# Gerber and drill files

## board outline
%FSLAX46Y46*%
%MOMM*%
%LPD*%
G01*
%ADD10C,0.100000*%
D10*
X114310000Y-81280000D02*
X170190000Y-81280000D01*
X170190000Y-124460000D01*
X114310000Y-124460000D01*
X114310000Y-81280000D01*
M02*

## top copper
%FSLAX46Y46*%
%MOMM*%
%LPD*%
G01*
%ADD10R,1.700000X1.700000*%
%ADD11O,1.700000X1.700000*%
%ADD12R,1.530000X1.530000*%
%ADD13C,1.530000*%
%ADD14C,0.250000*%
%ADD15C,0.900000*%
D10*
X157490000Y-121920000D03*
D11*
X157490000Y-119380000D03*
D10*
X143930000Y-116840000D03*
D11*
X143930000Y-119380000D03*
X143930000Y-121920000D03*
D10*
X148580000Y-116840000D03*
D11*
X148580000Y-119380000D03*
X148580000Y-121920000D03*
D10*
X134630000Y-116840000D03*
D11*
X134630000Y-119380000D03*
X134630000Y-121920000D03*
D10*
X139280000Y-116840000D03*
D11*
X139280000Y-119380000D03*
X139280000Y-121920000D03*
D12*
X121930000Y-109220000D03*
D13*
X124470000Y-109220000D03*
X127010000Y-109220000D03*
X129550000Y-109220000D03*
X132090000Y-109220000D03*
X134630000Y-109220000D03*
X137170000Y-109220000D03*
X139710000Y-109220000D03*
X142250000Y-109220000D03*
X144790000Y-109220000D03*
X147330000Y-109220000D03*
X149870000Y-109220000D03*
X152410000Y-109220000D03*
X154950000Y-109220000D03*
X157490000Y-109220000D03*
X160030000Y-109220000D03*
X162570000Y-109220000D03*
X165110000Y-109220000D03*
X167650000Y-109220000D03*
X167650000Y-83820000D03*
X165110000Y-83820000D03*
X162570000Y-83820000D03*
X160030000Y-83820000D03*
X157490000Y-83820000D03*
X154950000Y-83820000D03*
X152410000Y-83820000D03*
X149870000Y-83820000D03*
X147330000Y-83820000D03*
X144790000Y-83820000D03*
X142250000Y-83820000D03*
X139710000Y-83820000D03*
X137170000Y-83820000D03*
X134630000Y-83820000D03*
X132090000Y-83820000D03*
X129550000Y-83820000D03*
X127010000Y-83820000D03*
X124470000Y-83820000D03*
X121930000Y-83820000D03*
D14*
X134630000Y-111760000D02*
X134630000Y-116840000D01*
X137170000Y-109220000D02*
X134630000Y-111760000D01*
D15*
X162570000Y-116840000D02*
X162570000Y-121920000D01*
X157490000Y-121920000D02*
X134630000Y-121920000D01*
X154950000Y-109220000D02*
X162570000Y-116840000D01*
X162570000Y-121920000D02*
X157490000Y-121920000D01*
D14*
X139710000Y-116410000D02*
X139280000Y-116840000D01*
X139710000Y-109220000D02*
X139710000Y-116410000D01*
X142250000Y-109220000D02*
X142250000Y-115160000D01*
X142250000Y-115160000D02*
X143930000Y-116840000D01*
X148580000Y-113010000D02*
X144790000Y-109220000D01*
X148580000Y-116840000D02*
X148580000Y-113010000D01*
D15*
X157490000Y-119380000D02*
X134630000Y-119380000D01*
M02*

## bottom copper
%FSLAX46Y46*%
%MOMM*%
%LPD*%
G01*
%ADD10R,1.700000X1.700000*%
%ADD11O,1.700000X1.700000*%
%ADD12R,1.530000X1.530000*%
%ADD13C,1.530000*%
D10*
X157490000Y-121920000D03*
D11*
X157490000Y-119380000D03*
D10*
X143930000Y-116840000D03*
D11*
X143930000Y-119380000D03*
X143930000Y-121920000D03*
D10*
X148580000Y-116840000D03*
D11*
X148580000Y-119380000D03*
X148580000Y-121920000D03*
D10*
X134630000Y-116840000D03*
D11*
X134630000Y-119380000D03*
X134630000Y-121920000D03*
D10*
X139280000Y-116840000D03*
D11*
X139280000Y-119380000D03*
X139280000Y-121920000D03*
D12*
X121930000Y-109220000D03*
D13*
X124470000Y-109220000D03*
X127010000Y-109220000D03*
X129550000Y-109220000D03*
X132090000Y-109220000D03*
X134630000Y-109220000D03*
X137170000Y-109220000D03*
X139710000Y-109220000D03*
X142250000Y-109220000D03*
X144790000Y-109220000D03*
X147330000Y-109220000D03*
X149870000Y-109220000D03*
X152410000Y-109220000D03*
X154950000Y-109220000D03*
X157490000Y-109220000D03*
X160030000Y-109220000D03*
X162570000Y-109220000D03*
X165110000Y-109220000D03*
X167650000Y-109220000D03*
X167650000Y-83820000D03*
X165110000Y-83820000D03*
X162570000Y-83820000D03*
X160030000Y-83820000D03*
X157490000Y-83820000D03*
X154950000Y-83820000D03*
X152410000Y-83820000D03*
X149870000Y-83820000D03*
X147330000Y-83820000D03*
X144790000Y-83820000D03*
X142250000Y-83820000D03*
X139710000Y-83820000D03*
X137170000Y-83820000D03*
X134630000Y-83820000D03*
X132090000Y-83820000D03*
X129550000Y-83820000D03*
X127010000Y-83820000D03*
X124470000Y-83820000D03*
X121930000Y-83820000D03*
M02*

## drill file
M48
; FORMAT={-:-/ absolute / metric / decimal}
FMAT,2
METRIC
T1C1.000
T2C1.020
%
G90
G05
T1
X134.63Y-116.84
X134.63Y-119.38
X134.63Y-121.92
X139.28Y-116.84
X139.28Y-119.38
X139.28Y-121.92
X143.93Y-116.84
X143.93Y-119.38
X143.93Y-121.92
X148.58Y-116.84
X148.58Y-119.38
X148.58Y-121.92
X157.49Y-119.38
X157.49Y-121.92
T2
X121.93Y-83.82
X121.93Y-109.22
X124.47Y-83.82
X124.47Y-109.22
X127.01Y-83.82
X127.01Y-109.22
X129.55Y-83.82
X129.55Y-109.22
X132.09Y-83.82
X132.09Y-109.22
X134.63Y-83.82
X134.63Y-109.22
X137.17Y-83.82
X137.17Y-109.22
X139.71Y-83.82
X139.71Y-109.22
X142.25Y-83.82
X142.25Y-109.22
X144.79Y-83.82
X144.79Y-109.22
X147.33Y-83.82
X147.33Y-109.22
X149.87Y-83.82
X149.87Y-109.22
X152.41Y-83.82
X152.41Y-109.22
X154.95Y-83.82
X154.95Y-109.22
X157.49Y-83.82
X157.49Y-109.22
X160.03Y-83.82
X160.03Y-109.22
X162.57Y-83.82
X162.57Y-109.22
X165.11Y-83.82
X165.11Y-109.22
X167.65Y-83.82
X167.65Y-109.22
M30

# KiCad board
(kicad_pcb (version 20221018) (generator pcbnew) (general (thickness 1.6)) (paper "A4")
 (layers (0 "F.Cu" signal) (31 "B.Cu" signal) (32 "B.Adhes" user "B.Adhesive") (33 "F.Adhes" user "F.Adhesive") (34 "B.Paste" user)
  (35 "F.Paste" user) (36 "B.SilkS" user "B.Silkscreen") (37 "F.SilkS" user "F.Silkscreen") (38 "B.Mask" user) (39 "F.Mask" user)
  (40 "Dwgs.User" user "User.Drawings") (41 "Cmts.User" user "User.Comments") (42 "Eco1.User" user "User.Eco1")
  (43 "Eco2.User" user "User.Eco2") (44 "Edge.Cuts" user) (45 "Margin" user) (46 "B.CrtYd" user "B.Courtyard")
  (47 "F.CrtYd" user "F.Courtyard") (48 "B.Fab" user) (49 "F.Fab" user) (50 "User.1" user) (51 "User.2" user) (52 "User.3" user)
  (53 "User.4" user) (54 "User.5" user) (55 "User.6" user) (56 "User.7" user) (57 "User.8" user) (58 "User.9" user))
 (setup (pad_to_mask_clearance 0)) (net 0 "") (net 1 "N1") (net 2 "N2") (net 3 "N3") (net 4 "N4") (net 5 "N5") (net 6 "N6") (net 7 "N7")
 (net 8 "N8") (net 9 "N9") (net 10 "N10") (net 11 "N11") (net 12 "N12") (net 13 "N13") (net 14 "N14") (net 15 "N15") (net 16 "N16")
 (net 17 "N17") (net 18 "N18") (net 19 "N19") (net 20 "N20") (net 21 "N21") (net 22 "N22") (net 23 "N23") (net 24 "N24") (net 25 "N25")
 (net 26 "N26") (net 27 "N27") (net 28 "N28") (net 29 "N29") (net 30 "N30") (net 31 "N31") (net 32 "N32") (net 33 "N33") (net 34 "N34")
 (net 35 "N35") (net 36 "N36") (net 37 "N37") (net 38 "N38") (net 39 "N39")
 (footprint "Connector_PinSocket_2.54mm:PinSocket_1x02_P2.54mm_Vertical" (layer "F.Cu") (at 157.49 121.92 180)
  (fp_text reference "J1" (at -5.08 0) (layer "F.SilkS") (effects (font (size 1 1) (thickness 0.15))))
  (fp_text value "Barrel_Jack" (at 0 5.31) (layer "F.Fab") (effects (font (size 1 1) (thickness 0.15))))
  (pad "1" thru_hole rect (at 0 0 180) (size 1.7 1.7) (drill 1) (layers "*.Cu" "*.Mask") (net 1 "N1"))
  (pad "2" thru_hole oval (at 0 2.54 180) (size 1.7 1.7) (drill 1) (layers "*.Cu" "*.Mask") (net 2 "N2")))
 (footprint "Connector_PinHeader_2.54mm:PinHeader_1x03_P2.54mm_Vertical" (layer "F.Cu") (at 143.93 116.84)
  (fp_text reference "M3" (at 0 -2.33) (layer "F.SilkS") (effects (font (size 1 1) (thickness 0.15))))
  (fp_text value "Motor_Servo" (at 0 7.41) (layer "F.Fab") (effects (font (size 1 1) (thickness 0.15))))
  (pad "1" thru_hole rect (at 0 0) (size 1.7 1.7) (drill 1) (layers "*.Cu" "*.Mask") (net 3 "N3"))
  (pad "2" thru_hole oval (at 0 2.54) (size 1.7 1.7) (drill 1) (layers "*.Cu" "*.Mask") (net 2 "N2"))
  (pad "3" thru_hole oval (at 0 5.08) (size 1.7 1.7) (drill 1) (layers "*.Cu" "*.Mask") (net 1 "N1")))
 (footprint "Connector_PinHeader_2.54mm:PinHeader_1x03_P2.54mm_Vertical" (layer "F.Cu") (at 148.58 116.84)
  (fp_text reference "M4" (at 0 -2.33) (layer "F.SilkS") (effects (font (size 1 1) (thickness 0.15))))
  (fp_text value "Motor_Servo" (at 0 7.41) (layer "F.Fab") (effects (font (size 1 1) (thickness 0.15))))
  (pad "1" thru_hole rect (at 0 0) (size 1.7 1.7) (drill 1) (layers "*.Cu" "*.Mask") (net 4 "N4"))
  (pad "2" thru_hole oval (at 0 2.54) (size 1.7 1.7) (drill 1) (layers "*.Cu" "*.Mask") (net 2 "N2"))
  (pad "3" thru_hole oval (at 0 5.08) (size 1.7 1.7) (drill 1) (layers "*.Cu" "*.Mask") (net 1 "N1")))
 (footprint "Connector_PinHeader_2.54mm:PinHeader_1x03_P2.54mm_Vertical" (layer "F.Cu") (at 134.63 116.84)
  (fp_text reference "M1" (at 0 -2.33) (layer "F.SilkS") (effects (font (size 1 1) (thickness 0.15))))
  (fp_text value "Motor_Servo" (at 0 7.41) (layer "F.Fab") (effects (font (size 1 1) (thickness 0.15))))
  (pad "1" thru_hole rect (at 0 0) (size 1.7 1.7) (drill 1) (layers "*.Cu" "*.Mask") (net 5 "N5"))
  (pad "2" thru_hole oval (at 0 2.54) (size 1.7 1.7) (drill 1) (layers "*.Cu" "*.Mask") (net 2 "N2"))
  (pad "3" thru_hole oval (at 0 5.08) (size 1.7 1.7) (drill 1) (layers "*.Cu" "*.Mask") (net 1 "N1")))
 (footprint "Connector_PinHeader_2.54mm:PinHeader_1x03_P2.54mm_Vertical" (layer "F.Cu") (at 139.28 116.84)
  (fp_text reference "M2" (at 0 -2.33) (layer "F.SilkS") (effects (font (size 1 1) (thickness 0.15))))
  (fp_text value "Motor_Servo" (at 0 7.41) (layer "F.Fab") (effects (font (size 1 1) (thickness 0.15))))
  (pad "1" thru_hole rect (at 0 0) (size 1.7 1.7) (drill 1) (layers "*.Cu" "*.Mask") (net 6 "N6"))
  (pad "2" thru_hole oval (at 0 2.54) (size 1.7 1.7) (drill 1) (layers "*.Cu" "*.Mask") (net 2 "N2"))
  (pad "3" thru_hole oval (at 0 5.08) (size 1.7 1.7) (drill 1) (layers "*.Cu" "*.Mask") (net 1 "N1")))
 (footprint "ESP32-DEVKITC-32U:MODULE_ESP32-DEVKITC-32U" (layer "F.Cu") (at 144.78 96.52 90)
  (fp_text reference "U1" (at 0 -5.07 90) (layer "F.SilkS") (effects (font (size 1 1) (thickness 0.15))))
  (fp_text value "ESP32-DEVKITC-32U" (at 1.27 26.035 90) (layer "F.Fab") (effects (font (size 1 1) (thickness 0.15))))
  (pad "1" thru_hole rect (at -12.7 -22.85 90) (size 1.53 1.53) (drill 1.02) (layers "*.Cu" "*.Mask") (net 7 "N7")
   (solder_mask_margin 0.102))
  (pad "2" thru_hole circle (at -12.7 -20.31 90) (size 1.53 1.53) (drill 1.02) (layers "*.Cu" "*.Mask") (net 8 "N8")
   (solder_mask_margin 0.102))
  (pad "3" thru_hole circle (at -12.7 -17.77 90) (size 1.53 1.53) (drill 1.02) (layers "*.Cu" "*.Mask") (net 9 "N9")
   (solder_mask_margin 0.102))
  (pad "4" thru_hole circle (at -12.7 -15.23 90) (size 1.53 1.53) (drill 1.02) (layers "*.Cu" "*.Mask") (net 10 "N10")
   (solder_mask_margin 0.102))
  (pad "5" thru_hole circle (at -12.7 -12.69 90) (size 1.53 1.53) (drill 1.02) (layers "*.Cu" "*.Mask") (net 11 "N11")
   (solder_mask_margin 0.102))
  (pad "6" thru_hole circle (at -12.7 -10.15 90) (size 1.53 1.53) (drill 1.02) (layers "*.Cu" "*.Mask") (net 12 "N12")
   (solder_mask_margin 0.102))
  (pad "7" thru_hole circle (at -12.7 -7.61 90) (size 1.53 1.53) (drill 1.02) (layers "*.Cu" "*.Mask") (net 5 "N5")
   (solder_mask_margin 0.102))
  (pad "8" thru_hole circle (at -12.7 -5.07 90) (size 1.53 1.53) (drill 1.02) (layers "*.Cu" "*.Mask") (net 6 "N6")
   (solder_mask_margin 0.102))
  (pad "9" thru_hole circle (at -12.7 -2.53 90) (size 1.53 1.53) (drill 1.02) (layers "*.Cu" "*.Mask") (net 3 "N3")
   (solder_mask_margin 0.102))
  (pad "10" thru_hole circle (at -12.7 0.01 90) (size 1.53 1.53) (drill 1.02) (layers "*.Cu" "*.Mask") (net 4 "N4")
   (solder_mask_margin 0.102))
  (pad "11" thru_hole circle (at -12.7 2.55 90) (size 1.53 1.53) (drill 1.02) (layers "*.Cu" "*.Mask") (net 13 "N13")
   (solder_mask_margin 0.102))
  (pad "12" thru_hole circle (at -12.7 5.09 90) (size 1.53 1.53) (drill 1.02) (layers "*.Cu" "*.Mask") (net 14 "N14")
   (solder_mask_margin 0.102))
  (pad "13" thru_hole circle (at -12.7 7.63 90) (size 1.53 1.53) (drill 1.02) (layers "*.Cu" "*.Mask") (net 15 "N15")
   (solder_mask_margin 0.102))
  (pad "14" thru_hole circle (at -12.7 10.17 90) (size 1.53 1.53) (drill 1.02) (layers "*.Cu" "*.Mask") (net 1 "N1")
   (solder_mask_margin 0.102))
  (pad "15" thru_hole circle (at -12.7 12.71 90) (size 1.53 1.53) (drill 1.02) (layers "*.Cu" "*.Mask") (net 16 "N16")
   (solder_mask_margin 0.102))
  (pad "16" thru_hole circle (at -12.7 15.25 90) (size 1.53 1.53) (drill 1.02) (layers "*.Cu" "*.Mask") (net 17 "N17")
   (solder_mask_margin 0.102))
  (pad "17" thru_hole circle (at -12.7 17.79 90) (size 1.53 1.53) (drill 1.02) (layers "*.Cu" "*.Mask") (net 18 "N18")
   (solder_mask_margin 0.102))
  (pad "18" thru_hole circle (at -12.7 20.33 90) (size 1.53 1.53) (drill 1.02) (layers "*.Cu" "*.Mask") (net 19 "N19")
   (solder_mask_margin 0.102))
  (pad "19" thru_hole circle (at -12.7 22.87 90) (size 1.53 1.53) (drill 1.02) (layers "*.Cu" "*.Mask") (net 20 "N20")
   (solder_mask_margin 0.102))
  (pad "20" thru_hole circle (at 12.7 22.87 90) (size 1.53 1.53) (drill 1.02) (layers "*.Cu" "*.Mask") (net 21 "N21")
   (solder_mask_margin 0.102))
  (pad "21" thru_hole circle (at 12.7 20.33 90) (size 1.53 1.53) (drill 1.02) (layers "*.Cu" "*.Mask") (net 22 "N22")
   (solder_mask_margin 0.102))
  (pad "22" thru_hole circle (at 12.7 17.79 90) (size 1.53 1.53) (drill 1.02) (layers "*.Cu" "*.Mask") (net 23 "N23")
   (solder_mask_margin 0.102))
  (pad "23" thru_hole circle (at 12.7 15.25 90) (size 1.53 1.53) (drill 1.02) (layers "*.Cu" "*.Mask") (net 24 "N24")
   (solder_mask_margin 0.102))
  (pad "24" thru_hole circle (at 12.7 12.71 90) (size 1.53 1.53) (drill 1.02) (layers "*.Cu" "*.Mask") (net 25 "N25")
   (solder_mask_margin 0.102))
  (pad "25" thru_hole circle (at 12.7 10.17 90) (size 1.53 1.53) (drill 1.02) (layers "*.Cu" "*.Mask") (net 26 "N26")
   (solder_mask_margin 0.102))
  (pad "26" thru_hole circle (at 12.7 7.63 90) (size 1.53 1.53) (drill 1.02) (layers "*.Cu" "*.Mask") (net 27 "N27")
   (solder_mask_margin 0.102))
  (pad "27" thru_hole circle (at 12.7 5.09 90) (size 1.53 1.53) (drill 1.02) (layers "*.Cu" "*.Mask") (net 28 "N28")
   (solder_mask_margin 0.102))
  (pad "28" thru_hole circle (at 12.7 2.55 90) (size 1.53 1.53) (drill 1.02) (layers "*.Cu" "*.Mask") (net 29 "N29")
   (solder_mask_margin 0.102))
  (pad "29" thru_hole circle (at 12.7 0.01 90) (size 1.53 1.53) (drill 1.02) (layers "*.Cu" "*.Mask") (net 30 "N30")
   (solder_mask_margin 0.102))
  (pad "30" thru_hole circle (at 12.7 -2.53 90) (size 1.53 1.53) (drill 1.02) (layers "*.Cu" "*.Mask") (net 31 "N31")
   (solder_mask_margin 0.102))
  (pad "31" thru_hole circle (at 12.7 -5.07 90) (size 1.53 1.53) (drill 1.02) (layers "*.Cu" "*.Mask") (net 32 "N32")
   (solder_mask_margin 0.102))
  (pad "32" thru_hole circle (at 12.7 -7.61 90) (size 1.53 1.53) (drill 1.02) (layers "*.Cu" "*.Mask") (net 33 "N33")
   (solder_mask_margin 0.102))
  (pad "33" thru_hole circle (at 12.7 -10.15 90) (size 1.53 1.53) (drill 1.02) (layers "*.Cu" "*.Mask") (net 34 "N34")
   (solder_mask_margin 0.102))
  (pad "34" thru_hole circle (at 12.7 -12.69 90) (size 1.53 1.53) (drill 1.02) (layers "*.Cu" "*.Mask") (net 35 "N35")
   (solder_mask_margin 0.102))
  (pad "35" thru_hole circle (at 12.7 -15.23 90) (size 1.53 1.53) (drill 1.02) (layers "*.Cu" "*.Mask") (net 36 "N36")
   (solder_mask_margin 0.102))
  (pad "36" thru_hole circle (at 12.7 -17.77 90) (size 1.53 1.53) (drill 1.02) (layers "*.Cu" "*.Mask") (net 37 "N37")
   (solder_mask_margin 0.102))
  (pad "37" thru_hole circle (at 12.7 -20.31 90) (size 1.53 1.53) (drill 1.02) (layers "*.Cu" "*.Mask") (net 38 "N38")
   (solder_mask_margin 0.102))
  (pad "38" thru_hole circle (at 12.7 -22.85 90) (size 1.53 1.53) (drill 1.02) (layers "*.Cu" "*.Mask") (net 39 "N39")
   (solder_mask_margin 0.102)))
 (gr_rect (start 114.31 81.28) (end 170.19 124.46) (stroke (width 0.1) (type default)) (fill none) (layer "Edge.Cuts"))
 (segment (start 134.63 111.76) (end 134.63 116.84) (width 0.25) (layer "F.Cu") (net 5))
 (segment (start 137.17 109.22) (end 134.63 111.76) (width 0.25) (layer "F.Cu") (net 5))
 (segment (start 162.57 116.84) (end 162.57 121.92) (width 0.9) (layer "F.Cu") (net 1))
 (segment (start 157.49 121.92) (end 134.63 121.92) (width 0.9) (layer "F.Cu") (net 1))
 (segment (start 154.95 109.22) (end 162.57 116.84) (width 0.9) (layer "F.Cu") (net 1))
 (segment (start 162.57 121.92) (end 157.49 121.92) (width 0.9) (layer "F.Cu") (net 1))
 (segment (start 139.71 116.41) (end 139.28 116.84) (width 0.25) (layer "F.Cu") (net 6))
 (segment (start 139.71 109.22) (end 139.71 116.41) (width 0.25) (layer "F.Cu") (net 6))
 (segment (start 142.25 109.22) (end 142.25 115.16) (width 0.25) (layer "F.Cu") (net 3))
 (segment (start 142.25 115.16) (end 143.93 116.84) (width 0.25) (layer "F.Cu") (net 3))
 (segment (start 148.58 113.01) (end 144.79 109.22) (width 0.25) (layer "F.Cu") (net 4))
 (segment (start 148.58 116.84) (end 148.58 113.01) (width 0.25) (layer "F.Cu") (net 4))
 (segment (start 157.49 119.38) (end 134.63 119.38) (width 0.9) (layer "F.Cu") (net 2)))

